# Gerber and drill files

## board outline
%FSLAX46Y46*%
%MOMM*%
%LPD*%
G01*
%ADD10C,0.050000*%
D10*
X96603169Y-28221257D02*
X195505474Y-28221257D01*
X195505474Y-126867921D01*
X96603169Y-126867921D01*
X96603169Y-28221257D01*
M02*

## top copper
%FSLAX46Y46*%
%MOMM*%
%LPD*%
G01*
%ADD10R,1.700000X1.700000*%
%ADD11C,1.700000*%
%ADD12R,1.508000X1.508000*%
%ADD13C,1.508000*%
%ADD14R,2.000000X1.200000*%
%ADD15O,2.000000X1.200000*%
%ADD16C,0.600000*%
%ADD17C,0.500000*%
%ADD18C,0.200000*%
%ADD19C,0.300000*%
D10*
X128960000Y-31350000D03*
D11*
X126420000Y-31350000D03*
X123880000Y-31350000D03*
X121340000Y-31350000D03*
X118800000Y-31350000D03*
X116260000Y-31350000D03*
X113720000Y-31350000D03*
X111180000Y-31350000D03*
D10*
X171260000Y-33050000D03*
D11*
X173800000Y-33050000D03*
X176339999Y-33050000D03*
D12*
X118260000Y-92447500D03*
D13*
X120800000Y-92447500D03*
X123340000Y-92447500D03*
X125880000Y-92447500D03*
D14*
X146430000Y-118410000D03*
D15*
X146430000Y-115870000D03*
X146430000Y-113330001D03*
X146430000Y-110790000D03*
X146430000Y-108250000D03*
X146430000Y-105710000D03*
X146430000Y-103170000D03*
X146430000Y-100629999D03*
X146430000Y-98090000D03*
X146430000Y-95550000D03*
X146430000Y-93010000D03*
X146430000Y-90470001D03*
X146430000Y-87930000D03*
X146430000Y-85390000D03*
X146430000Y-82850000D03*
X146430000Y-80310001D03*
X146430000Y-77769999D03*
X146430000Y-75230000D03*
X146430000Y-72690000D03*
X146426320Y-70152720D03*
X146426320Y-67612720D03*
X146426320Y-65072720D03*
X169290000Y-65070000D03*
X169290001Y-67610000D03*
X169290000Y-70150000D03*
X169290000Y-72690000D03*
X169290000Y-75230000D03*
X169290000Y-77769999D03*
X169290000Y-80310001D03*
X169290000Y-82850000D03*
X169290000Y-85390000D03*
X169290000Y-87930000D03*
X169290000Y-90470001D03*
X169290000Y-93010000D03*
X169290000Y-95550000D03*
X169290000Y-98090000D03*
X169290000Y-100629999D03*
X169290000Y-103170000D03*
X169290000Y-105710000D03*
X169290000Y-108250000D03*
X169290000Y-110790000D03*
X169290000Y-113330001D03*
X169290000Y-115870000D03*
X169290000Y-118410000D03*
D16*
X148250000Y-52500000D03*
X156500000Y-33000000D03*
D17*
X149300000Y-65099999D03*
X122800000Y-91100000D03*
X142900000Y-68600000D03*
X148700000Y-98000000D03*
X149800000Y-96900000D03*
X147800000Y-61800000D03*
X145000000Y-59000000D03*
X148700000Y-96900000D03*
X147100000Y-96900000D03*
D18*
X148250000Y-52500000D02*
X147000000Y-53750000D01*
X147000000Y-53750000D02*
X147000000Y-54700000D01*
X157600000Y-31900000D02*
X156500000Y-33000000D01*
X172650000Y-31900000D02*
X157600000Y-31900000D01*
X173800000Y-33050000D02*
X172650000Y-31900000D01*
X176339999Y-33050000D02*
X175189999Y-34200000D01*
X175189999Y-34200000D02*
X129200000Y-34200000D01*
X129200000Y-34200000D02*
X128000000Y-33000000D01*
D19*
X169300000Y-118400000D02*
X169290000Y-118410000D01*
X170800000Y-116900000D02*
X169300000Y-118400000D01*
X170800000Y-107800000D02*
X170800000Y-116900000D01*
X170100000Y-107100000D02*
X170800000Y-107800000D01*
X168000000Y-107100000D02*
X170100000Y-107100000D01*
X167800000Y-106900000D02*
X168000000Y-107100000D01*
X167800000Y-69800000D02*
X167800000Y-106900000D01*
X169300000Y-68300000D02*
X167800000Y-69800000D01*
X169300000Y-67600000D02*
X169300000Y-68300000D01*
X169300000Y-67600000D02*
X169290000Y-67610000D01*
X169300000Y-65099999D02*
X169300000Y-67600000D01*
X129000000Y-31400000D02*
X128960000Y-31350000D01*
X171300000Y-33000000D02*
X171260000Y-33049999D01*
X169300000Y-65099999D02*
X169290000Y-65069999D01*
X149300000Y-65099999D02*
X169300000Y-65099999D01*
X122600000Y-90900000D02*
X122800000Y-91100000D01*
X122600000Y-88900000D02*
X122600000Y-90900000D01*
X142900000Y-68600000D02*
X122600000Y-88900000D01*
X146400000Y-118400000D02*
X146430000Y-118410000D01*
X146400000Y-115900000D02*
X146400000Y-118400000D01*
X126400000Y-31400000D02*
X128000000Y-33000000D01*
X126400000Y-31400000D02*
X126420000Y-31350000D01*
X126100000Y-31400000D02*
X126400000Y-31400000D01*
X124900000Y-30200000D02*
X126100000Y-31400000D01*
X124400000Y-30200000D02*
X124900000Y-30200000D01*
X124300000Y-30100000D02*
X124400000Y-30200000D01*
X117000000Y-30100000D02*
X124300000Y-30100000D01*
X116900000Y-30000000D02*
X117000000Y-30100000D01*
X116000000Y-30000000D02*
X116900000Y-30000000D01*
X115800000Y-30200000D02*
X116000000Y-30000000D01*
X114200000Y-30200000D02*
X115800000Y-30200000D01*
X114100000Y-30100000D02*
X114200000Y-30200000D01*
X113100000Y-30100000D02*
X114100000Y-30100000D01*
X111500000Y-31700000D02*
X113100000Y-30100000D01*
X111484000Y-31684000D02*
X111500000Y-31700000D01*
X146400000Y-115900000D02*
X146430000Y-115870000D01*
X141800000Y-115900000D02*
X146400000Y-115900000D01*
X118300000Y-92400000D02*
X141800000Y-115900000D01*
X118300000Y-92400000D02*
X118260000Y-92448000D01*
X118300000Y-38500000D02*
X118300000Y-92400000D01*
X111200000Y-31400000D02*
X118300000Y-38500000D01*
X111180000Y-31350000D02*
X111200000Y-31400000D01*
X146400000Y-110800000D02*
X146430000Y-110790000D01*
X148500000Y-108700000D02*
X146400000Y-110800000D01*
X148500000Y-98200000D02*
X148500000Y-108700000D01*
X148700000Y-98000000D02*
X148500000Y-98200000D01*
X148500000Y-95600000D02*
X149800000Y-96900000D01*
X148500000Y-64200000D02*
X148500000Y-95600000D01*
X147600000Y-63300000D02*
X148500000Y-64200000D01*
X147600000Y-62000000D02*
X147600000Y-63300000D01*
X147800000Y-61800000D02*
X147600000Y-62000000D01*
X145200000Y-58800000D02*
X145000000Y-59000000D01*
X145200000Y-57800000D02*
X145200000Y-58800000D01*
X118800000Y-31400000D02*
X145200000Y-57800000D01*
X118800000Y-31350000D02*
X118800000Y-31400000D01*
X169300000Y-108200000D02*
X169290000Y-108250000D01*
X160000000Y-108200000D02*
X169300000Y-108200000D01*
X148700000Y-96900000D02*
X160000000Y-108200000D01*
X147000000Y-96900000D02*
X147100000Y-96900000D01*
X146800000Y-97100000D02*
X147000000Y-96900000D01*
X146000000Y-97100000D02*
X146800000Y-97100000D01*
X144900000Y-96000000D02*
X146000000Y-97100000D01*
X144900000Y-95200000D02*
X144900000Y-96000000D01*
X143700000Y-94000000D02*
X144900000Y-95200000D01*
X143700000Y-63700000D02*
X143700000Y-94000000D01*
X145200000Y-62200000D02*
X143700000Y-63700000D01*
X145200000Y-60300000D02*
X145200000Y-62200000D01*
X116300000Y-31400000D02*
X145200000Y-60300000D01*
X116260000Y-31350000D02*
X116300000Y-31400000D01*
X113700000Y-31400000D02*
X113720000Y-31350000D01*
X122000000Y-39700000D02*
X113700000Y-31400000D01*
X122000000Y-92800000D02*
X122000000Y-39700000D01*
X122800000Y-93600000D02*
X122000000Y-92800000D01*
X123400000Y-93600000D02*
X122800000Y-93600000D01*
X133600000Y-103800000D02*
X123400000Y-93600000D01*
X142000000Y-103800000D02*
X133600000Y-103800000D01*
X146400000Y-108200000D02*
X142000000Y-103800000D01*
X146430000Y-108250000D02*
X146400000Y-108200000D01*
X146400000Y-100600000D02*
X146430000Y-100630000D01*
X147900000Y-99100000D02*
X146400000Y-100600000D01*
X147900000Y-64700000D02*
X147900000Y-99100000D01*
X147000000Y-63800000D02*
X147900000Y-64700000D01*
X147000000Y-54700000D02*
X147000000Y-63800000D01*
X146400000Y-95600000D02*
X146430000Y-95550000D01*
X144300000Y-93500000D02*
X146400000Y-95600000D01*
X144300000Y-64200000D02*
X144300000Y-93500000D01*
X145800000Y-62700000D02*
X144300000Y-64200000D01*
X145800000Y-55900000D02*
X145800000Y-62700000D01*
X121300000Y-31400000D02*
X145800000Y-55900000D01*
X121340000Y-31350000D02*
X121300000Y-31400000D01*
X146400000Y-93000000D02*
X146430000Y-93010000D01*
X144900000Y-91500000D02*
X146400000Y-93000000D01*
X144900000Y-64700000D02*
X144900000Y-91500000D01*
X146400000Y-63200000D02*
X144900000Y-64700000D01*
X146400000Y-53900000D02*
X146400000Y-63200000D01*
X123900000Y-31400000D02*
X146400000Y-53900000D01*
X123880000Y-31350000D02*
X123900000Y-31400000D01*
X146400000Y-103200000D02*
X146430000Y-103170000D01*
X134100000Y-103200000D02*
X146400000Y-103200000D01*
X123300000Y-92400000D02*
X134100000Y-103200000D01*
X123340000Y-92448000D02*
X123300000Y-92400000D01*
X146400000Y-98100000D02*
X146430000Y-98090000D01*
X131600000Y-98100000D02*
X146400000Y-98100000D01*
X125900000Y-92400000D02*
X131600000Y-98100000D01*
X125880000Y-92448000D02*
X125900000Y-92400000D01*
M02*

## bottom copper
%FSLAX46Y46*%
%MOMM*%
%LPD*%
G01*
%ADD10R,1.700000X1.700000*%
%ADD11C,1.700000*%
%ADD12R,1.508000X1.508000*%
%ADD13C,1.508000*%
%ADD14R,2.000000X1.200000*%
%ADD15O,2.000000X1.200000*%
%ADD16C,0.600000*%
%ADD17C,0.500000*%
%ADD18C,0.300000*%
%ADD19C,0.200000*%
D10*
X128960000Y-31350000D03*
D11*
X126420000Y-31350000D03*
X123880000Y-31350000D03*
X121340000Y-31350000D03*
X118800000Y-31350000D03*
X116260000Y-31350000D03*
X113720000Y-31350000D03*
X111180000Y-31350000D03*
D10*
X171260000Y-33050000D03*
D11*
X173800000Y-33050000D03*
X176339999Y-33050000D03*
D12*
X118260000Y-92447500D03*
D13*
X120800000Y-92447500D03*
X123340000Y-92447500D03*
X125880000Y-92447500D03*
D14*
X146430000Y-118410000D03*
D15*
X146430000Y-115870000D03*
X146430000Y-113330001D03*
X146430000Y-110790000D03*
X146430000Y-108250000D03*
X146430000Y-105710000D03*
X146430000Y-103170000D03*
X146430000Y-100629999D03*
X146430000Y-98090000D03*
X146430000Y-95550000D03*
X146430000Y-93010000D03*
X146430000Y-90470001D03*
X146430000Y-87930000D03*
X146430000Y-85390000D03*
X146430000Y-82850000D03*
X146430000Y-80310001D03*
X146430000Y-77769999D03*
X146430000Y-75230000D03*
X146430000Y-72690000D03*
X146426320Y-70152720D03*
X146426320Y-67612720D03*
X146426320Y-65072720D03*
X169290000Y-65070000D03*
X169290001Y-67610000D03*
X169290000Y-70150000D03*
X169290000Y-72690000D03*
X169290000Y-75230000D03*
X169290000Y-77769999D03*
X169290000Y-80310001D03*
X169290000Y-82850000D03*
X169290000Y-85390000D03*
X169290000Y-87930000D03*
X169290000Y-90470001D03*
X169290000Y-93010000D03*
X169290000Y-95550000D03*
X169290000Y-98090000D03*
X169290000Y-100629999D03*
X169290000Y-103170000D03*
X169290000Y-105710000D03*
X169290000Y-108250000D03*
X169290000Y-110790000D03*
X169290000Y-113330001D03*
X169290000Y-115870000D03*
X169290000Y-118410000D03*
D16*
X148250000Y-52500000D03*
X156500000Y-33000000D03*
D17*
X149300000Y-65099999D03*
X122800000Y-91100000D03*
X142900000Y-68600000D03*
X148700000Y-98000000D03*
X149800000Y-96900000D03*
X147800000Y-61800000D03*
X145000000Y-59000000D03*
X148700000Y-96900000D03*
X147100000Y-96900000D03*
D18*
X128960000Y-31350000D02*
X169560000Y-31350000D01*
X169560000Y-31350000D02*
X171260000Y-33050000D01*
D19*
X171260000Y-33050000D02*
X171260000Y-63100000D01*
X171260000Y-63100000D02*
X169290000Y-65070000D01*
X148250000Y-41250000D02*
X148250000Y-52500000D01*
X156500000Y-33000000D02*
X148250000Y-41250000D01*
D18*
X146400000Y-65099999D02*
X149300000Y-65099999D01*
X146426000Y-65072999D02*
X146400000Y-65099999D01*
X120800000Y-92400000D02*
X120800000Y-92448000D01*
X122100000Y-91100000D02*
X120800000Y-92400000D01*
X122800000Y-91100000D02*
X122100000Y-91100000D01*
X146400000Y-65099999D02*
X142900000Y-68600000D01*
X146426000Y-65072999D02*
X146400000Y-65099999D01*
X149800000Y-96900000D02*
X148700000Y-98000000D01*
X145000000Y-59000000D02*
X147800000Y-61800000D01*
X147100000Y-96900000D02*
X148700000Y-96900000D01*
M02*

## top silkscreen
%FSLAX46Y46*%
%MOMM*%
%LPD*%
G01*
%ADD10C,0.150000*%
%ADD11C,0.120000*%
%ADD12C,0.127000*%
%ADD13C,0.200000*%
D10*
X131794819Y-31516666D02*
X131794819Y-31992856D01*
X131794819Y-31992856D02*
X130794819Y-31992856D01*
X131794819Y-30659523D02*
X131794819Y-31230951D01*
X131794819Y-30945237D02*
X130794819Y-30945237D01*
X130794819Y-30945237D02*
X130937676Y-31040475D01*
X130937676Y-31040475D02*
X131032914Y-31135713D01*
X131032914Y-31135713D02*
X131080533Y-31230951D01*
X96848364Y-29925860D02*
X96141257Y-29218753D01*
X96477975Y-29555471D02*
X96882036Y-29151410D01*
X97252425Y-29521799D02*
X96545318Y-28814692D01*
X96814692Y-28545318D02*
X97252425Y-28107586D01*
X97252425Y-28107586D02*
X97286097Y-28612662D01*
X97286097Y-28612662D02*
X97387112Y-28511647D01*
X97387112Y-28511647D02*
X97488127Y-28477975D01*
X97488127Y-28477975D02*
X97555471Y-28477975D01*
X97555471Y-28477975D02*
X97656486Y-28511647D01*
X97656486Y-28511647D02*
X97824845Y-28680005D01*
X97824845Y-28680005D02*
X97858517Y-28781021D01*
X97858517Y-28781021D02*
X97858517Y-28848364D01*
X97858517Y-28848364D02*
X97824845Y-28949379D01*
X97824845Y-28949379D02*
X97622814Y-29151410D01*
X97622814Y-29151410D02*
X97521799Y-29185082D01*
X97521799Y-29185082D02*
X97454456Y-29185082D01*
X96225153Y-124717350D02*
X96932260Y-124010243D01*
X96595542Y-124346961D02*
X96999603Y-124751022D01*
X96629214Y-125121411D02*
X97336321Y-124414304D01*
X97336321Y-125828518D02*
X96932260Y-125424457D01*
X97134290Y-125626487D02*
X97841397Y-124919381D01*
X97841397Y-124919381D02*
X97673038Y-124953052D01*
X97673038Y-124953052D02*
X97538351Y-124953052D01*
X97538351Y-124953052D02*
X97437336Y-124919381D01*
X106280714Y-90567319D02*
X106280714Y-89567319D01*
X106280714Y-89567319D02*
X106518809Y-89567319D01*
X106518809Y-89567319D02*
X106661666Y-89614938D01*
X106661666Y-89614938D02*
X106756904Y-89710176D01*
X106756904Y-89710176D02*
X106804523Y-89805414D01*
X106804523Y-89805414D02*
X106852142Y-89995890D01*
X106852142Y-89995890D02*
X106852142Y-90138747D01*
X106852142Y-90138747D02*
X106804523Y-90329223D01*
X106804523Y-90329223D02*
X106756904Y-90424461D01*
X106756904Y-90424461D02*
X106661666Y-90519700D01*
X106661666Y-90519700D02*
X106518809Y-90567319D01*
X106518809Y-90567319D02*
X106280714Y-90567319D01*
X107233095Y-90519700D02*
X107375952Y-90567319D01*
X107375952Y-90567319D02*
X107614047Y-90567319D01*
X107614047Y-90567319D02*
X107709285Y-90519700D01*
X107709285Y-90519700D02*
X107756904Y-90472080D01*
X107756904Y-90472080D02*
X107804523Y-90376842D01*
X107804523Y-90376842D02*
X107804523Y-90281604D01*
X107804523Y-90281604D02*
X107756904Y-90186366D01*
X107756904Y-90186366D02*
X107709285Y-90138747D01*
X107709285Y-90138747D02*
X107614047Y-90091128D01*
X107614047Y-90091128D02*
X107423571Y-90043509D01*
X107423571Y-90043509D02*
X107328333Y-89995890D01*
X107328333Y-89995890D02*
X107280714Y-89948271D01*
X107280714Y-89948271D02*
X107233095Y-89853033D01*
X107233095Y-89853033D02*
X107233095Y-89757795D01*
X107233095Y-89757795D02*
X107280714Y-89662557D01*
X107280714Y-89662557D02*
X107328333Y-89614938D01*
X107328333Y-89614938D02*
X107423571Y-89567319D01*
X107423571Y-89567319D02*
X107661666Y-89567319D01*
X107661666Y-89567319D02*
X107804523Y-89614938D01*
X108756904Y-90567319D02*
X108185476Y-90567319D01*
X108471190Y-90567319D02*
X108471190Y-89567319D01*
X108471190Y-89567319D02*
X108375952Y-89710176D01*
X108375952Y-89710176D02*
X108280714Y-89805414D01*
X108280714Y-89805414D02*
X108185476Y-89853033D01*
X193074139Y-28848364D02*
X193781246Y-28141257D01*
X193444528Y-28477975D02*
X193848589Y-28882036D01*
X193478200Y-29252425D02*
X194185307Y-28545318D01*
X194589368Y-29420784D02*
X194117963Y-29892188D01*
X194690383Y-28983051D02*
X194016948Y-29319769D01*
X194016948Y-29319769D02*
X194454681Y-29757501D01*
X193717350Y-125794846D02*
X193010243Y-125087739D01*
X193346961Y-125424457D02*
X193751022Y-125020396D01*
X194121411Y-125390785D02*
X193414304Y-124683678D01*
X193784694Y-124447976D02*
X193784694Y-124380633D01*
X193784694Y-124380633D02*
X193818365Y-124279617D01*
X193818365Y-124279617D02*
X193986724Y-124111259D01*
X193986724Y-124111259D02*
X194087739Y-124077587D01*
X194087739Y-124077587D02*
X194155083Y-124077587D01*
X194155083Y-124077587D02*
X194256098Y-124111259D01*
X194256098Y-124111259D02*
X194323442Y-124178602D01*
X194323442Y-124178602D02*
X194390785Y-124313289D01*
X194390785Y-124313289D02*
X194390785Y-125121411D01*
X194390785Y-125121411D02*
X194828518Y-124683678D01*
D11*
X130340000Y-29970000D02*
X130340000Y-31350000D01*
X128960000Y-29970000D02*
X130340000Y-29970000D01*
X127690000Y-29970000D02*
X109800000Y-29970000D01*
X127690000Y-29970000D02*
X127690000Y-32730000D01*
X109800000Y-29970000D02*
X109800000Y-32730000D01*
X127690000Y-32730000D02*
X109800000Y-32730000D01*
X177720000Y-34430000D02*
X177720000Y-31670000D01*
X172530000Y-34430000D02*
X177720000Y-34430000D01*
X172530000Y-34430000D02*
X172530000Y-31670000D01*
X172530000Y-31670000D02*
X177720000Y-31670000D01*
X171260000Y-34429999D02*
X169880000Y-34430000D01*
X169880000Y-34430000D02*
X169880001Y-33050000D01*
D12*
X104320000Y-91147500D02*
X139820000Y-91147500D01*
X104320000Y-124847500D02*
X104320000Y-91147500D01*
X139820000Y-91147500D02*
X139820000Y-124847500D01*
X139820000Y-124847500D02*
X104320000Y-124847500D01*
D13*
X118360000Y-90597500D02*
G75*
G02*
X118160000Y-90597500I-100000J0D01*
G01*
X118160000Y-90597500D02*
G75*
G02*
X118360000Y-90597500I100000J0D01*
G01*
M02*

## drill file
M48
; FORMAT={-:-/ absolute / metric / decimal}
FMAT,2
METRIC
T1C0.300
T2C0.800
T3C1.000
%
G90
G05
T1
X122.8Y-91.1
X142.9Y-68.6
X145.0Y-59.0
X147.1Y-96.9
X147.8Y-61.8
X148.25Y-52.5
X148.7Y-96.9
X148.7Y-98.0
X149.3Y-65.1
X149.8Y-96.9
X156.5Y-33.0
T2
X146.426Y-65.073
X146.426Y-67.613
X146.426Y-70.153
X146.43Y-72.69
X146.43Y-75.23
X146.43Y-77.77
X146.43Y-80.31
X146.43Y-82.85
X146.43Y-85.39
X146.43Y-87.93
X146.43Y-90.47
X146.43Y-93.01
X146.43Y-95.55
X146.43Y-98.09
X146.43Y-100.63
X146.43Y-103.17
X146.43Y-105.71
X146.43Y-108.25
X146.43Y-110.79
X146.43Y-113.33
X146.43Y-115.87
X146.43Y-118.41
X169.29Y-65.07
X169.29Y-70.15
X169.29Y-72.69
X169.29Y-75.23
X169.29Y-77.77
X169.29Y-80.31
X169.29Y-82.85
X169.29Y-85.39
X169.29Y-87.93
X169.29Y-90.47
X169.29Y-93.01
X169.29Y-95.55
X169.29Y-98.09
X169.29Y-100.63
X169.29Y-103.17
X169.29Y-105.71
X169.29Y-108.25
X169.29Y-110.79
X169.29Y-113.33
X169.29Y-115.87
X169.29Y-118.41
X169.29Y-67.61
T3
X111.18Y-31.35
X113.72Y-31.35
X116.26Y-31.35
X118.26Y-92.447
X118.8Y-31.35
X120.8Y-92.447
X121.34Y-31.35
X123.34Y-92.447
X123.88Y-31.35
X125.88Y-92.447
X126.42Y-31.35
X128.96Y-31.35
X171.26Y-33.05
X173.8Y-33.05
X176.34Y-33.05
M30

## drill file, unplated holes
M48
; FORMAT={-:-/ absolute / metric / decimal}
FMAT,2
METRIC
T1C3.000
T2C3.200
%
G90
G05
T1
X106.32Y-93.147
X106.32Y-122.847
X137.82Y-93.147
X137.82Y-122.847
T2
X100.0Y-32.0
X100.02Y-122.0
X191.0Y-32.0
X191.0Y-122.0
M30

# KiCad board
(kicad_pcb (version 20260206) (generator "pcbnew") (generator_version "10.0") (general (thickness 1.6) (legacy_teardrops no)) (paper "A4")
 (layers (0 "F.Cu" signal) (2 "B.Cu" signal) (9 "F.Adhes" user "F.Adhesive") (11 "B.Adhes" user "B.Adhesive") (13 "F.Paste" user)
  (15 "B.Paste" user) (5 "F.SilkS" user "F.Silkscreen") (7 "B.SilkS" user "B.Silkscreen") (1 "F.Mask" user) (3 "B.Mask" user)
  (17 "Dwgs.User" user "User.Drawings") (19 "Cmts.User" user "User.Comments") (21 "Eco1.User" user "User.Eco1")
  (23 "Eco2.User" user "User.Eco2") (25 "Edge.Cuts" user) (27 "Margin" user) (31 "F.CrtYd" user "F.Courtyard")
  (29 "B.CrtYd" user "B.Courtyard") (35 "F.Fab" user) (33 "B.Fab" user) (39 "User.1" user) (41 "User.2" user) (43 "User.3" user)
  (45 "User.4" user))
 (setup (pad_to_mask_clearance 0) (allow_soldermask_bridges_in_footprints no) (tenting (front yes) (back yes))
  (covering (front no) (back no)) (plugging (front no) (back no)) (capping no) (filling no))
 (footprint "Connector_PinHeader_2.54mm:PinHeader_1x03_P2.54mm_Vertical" (layer "F.Cu") (at 171.26 33.05 90)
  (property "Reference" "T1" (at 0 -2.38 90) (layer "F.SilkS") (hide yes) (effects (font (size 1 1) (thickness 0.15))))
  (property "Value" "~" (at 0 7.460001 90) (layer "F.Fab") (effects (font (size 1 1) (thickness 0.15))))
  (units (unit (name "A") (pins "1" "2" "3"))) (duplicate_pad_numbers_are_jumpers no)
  (fp_line (start -1.38 -1.38) (end 0 -1.379999) (stroke (width 0.12) (type solid)) (layer "F.SilkS"))
  (fp_line (start -1.379999 0) (end -1.38 -1.38) (stroke (width 0.12) (type solid)) (layer "F.SilkS"))
  (fp_line (start 1.38 1.27) (end 1.38 6.46) (stroke (width 0.12) (type solid)) (layer "F.SilkS"))
  (fp_line (start -1.38 1.27) (end 1.38 1.27) (stroke (width 0.12) (type solid)) (layer "F.SilkS"))
  (fp_line (start -1.38 1.27) (end -1.38 6.46) (stroke (width 0.12) (type solid)) (layer "F.SilkS"))
  (fp_line (start -1.38 6.46) (end 1.38 6.46) (stroke (width 0.12) (type solid)) (layer "F.SilkS"))
  (pad "1" thru_hole rect (at 0 0 90) (size 1.7 1.7) (drill 1) (layers "*.Cu" "*.Mask") (remove_unused_layers no) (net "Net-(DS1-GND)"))
  (pad "2" thru_hole circle (at 0 2.54 90) (size 1.7 1.7) (drill 1) (layers "*.Cu" "*.Mask") (remove_unused_layers no) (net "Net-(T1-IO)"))
  (pad "3" thru_hole circle (at 0 5.079999 90) (size 1.7 1.7) (drill 1) (layers "*.Cu" "*.Mask") (remove_unused_layers no)
   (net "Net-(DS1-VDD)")))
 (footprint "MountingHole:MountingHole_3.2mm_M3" (layer "F.Cu") (at 100 32 45)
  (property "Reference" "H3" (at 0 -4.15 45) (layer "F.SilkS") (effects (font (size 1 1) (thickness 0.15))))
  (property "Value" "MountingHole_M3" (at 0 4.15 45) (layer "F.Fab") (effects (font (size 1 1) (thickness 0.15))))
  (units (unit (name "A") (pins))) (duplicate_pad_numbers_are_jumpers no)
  (pad "" np_thru_hole circle (at 0 0 45) (size 3.2 3.2) (drill 3.2) (layers "*.Cu" "*.Mask")))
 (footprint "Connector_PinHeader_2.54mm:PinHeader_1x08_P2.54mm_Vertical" (layer "F.Cu") (at 128.96 31.35 -90)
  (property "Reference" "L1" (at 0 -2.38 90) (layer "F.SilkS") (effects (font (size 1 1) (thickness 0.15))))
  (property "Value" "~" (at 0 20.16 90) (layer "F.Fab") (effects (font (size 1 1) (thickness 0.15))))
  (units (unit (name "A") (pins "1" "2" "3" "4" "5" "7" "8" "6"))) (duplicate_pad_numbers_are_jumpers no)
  (fp_line (start -1.38 19.16) (end 1.38 19.16) (stroke (width 0.12) (type solid)) (layer "F.SilkS"))
  (fp_line (start -1.38 1.27) (end -1.38 19.16) (stroke (width 0.12) (type solid)) (layer "F.SilkS"))
  (fp_line (start -1.38 1.27) (end 1.38 1.27) (stroke (width 0.12) (type solid)) (layer "F.SilkS"))
  (fp_line (start 1.38 1.27) (end 1.38 19.16) (stroke (width 0.12) (type solid)) (layer "F.SilkS"))
  (fp_line (start -1.38 0) (end -1.38 -1.38) (stroke (width 0.12) (type solid)) (layer "F.SilkS"))
  (fp_line (start -1.38 -1.38) (end 0 -1.38) (stroke (width 0.12) (type solid)) (layer "F.SilkS"))
  (pad "1" thru_hole rect (at 0 0 270) (size 1.7 1.7) (drill 1) (layers "*.Cu" "*.Mask") (remove_unused_layers no) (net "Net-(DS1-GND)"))
  (pad "2" thru_hole circle (at 0 2.54 270) (size 1.7 1.7) (drill 1) (layers "*.Cu" "*.Mask") (remove_unused_layers no)
   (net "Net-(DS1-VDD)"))
  (pad "3" thru_hole circle (at 0 5.08 270) (size 1.7 1.7) (drill 1) (layers "*.Cu" "*.Mask") (remove_unused_layers no) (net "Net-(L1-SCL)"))
  (pad "4" thru_hole circle (at 0 7.62 270) (size 1.7 1.7) (drill 1) (layers "*.Cu" "*.Mask") (remove_unused_layers no) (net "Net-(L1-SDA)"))
  (pad "5" thru_hole circle (at 0 10.16 270) (size 1.7 1.7) (drill 1) (layers "*.Cu" "*.Mask") (remove_unused_layers no)
   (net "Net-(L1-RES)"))
  (pad "6" thru_hole circle (at 0 12.7 270) (size 1.7 1.7) (drill 1) (layers "*.Cu" "*.Mask") (remove_unused_layers no) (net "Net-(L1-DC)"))
  (pad "7" thru_hole circle (at 0 15.24 270) (size 1.7 1.7) (drill 1) (layers "*.Cu" "*.Mask") (remove_unused_layers no) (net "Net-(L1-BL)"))
  (pad "8" thru_hole circle (at 0 17.78 270) (size 1.7 1.7) (drill 1) (layers "*.Cu" "*.Mask") (remove_unused_layers no)
   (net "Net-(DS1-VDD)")))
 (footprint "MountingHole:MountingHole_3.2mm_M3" (layer "F.Cu") (at 100.02 122 135)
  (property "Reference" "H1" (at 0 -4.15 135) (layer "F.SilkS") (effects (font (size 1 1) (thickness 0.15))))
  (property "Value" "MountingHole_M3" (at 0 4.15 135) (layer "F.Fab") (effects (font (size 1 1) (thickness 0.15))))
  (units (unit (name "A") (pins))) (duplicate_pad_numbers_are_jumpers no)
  (pad "" np_thru_hole circle (at 0 0 135) (size 3.2 3.2) (drill 3.2) (layers "*.Cu" "*.Mask")))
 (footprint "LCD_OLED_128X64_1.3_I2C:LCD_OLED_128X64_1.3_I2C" (layer "F.Cu") (at 122.07 107.9975)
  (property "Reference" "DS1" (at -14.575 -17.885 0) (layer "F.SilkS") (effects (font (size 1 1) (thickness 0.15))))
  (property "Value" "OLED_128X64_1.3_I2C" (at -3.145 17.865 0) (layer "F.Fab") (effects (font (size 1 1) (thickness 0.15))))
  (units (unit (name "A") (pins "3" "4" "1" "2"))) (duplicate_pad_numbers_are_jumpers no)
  (fp_line (start -17.75 -16.85) (end 17.75 -16.85) (stroke (width 0.127) (type solid)) (layer "F.SilkS"))
  (fp_line (start -17.75 16.85) (end -17.75 -16.85) (stroke (width 0.127) (type solid)) (layer "F.SilkS"))
  (fp_line (start 17.75 -16.85) (end 17.75 16.85) (stroke (width 0.127) (type solid)) (layer "F.SilkS"))
  (fp_line (start 17.75 16.85) (end -17.75 16.85) (stroke (width 0.127) (type solid)) (layer "F.SilkS"))
  (fp_circle (center -3.81 -17.4) (end -3.71 -17.4) (stroke (width 0.2) (type solid)) (fill no) (layer "F.SilkS"))
  (pad "" np_thru_hole circle (at -15.75 -14.85) (size 3 3) (drill 3) (layers "*.Cu" "*.Mask"))
  (pad "" np_thru_hole circle (at -15.75 14.85) (size 3 3) (drill 3) (layers "*.Cu" "*.Mask"))
  (pad "" np_thru_hole circle (at 15.75 -14.85) (size 3 3) (drill 3) (layers "*.Cu" "*.Mask"))
  (pad "" np_thru_hole circle (at 15.75 14.85) (size 3 3) (drill 3) (layers "*.Cu" "*.Mask"))
  (pad "1" thru_hole rect (at -3.81 -15.55) (size 1.508 1.508) (drill 1) (layers "*.Cu" "*.Mask") (remove_unused_layers no)
   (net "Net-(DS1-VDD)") (solder_mask_margin 0.102))
  (pad "2" thru_hole circle (at -1.27 -15.55) (size 1.508 1.508) (drill 1) (layers "*.Cu" "*.Mask") (remove_unused_layers no)
   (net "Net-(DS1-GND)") (solder_mask_margin 0.102))
  (pad "3" thru_hole circle (at 1.27 -15.55) (size 1.508 1.508) (drill 1) (layers "*.Cu" "*.Mask") (remove_unused_layers no)
   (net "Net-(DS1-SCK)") (solder_mask_margin 0.102))
  (pad "4" thru_hole circle (at 3.81 -15.55) (size 1.508 1.508) (drill 1) (layers "*.Cu" "*.Mask") (remove_unused_layers no)
   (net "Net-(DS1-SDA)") (solder_mask_margin 0.102)))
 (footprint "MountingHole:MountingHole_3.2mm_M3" (layer "F.Cu") (at 191 32 -45)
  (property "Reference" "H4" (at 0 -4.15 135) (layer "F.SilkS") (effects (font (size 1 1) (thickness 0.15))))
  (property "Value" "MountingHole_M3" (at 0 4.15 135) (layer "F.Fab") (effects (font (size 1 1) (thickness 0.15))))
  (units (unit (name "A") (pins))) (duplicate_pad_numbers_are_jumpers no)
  (pad "" np_thru_hole circle (at 0 0 315) (size 3.2 3.2) (drill 3.2) (layers "*.Cu" "*.Mask")))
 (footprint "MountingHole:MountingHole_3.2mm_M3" (layer "F.Cu") (at 191 122 -135)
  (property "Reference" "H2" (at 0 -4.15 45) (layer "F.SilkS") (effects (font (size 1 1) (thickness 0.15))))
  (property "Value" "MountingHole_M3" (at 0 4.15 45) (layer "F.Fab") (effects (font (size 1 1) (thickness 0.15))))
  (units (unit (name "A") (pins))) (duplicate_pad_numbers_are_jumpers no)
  (pad "" np_thru_hole circle (at 0 0 225) (size 3.2 3.2) (drill 3.2) (layers "*.Cu" "*.Mask")))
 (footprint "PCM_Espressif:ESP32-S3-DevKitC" (layer "B.Cu") (at 146.43 118.41)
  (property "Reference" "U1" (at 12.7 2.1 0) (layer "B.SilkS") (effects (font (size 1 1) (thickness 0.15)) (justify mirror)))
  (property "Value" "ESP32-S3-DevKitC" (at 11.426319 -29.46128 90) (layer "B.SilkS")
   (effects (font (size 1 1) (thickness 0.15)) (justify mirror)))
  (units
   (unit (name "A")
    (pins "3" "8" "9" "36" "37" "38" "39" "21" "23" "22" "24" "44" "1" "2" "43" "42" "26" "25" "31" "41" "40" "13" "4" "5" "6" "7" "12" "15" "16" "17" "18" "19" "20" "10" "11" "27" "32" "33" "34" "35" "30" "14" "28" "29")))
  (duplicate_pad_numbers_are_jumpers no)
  (pad "1" thru_hole rect (at 0 0 90) (size 1.2 2) (drill 0.8) (layers "*.Cu" "*.Mask") (remove_unused_layers no) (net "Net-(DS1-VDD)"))
  (pad "2" thru_hole oval (at 0 -2.54 90) (size 1.2 2) (drill 0.8) (layers "*.Cu" "*.Mask") (remove_unused_layers no) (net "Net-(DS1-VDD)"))
  (pad "3" thru_hole oval (at 0 -5.079999 90) (size 1.2 2) (drill 0.8) (layers "*.Cu" "*.Mask") (remove_unused_layers no)
   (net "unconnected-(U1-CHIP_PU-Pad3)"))
  (pad "4" thru_hole oval (at 0 -7.62 90) (size 1.2 2) (drill 0.8) (layers "*.Cu" "*.Mask") (remove_unused_layers no) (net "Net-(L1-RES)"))
  (pad "5" thru_hole oval (at 0 -10.16 90) (size 1.2 2) (drill 0.8) (layers "*.Cu" "*.Mask") (remove_unused_layers no) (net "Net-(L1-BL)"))
  (pad "6" thru_hole oval (at 0 -12.7 90) (size 1.2 2) (drill 0.8) (layers "*.Cu" "*.Mask") (remove_unused_layers no)
   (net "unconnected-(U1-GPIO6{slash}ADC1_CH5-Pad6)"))
  (pad "7" thru_hole oval (at 0 -15.24 90) (size 1.2 2) (drill 0.8) (layers "*.Cu" "*.Mask") (remove_unused_layers no) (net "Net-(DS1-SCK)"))
  (pad "8" thru_hole oval (at 0 -17.780001 90) (size 1.2 2) (drill 0.8) (layers "*.Cu" "*.Mask") (remove_unused_layers no)
   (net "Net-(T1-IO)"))
  (pad "9" thru_hole oval (at 0 -20.32 90) (size 1.2 2) (drill 0.8) (layers "*.Cu" "*.Mask") (remove_unused_layers no) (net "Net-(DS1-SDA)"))
  (pad "10" thru_hole oval (at 0 -22.86 90) (size 1.2 2) (drill 0.8) (layers "*.Cu" "*.Mask") (remove_unused_layers no) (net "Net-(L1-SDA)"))
  (pad "11" thru_hole oval (at 0 -25.4 90) (size 1.2 2) (drill 0.8) (layers "*.Cu" "*.Mask") (remove_unused_layers no) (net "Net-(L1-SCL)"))
  (pad "12" thru_hole oval (at 0 -27.939999 90) (size 1.2 2) (drill 0.8) (layers "*.Cu" "*.Mask") (remove_unused_layers no)
   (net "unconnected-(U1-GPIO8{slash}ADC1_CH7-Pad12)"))
  (pad "13" thru_hole oval (at 0 -30.48 90) (size 1.2 2) (drill 0.8) (layers "*.Cu" "*.Mask") (remove_unused_layers no)
   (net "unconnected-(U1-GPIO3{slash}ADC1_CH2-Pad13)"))
  (pad "14" thru_hole oval (at 0 -33.02 90) (size 1.2 2) (drill 0.8) (layers "*.Cu" "*.Mask") (remove_unused_layers no)
   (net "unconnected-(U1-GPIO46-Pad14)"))
  (pad "15" thru_hole oval (at 0 -35.56 90) (size 1.2 2) (drill 0.8) (layers "*.Cu" "*.Mask") (remove_unused_layers no)
   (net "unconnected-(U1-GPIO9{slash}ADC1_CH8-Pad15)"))
  (pad "16" thru_hole oval (at 0 -38.099999 90) (size 1.2 2) (drill 0.8) (layers "*.Cu" "*.Mask") (remove_unused_layers no)
   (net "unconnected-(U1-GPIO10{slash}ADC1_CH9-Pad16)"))
  (pad "17" thru_hole oval (at 0 -40.640001 90) (size 1.2 2) (drill 0.8) (layers "*.Cu" "*.Mask") (remove_unused_layers no)
   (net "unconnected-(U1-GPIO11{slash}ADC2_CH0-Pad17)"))
  (pad "18" thru_hole oval (at 0 -43.18 90) (size 1.2 2) (drill 0.8) (layers "*.Cu" "*.Mask") (remove_unused_layers no)
   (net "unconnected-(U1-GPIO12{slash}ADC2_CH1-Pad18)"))
  (pad "19" thru_hole oval (at 0 -45.72 90) (size 1.2 2) (drill 0.8) (layers "*.Cu" "*.Mask") (remove_unused_layers no)
   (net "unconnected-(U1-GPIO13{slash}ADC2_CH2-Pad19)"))
  (pad "20" thru_hole oval (at -0.00368 -48.25728 90) (size 1.2 2) (drill 0.8) (layers "*.Cu" "*.Mask") (remove_unused_layers no)
   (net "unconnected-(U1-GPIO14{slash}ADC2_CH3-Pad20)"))
  (pad "21" thru_hole oval (at -0.00368 -50.79728 90) (size 1.2 2) (drill 0.8) (layers "*.Cu" "*.Mask") (remove_unused_layers no)
   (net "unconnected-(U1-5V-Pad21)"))
  (pad "22" thru_hole oval (at -0.00368 -53.33728 90) (size 1.2 2) (drill 0.8) (layers "*.Cu" "*.Mask") (remove_unused_layers no)
   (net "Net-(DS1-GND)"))
  (pad "23" thru_hole oval (at 22.86 -53.34 90) (size 1.2 2) (drill 0.8) (layers "*.Cu" "*.Mask") (remove_unused_layers no)
   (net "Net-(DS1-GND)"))
  (pad "24" thru_hole oval (at 22.860001 -50.8 90) (size 1.2 2) (drill 0.8) (layers "*.Cu" "*.Mask") (remove_unused_layers no)
   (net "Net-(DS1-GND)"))
  (pad "25" thru_hole oval (at 22.86 -48.26 90) (size 1.2 2) (drill 0.8) (layers "*.Cu" "*.Mask") (remove_unused_layers no)
   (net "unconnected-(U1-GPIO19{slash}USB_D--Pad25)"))
  (pad "26" thru_hole oval (at 22.86 -45.72 90) (size 1.2 2) (drill 0.8) (layers "*.Cu" "*.Mask") (remove_unused_layers no)
   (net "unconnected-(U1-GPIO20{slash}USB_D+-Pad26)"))
  (pad "27" thru_hole oval (at 22.86 -43.18 90) (size 1.2 2) (drill 0.8) (layers "*.Cu" "*.Mask") (remove_unused_layers no)
   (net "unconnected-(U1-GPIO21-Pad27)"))
  (pad "28" thru_hole oval (at 22.86 -40.640001 90) (size 1.2 2) (drill 0.8) (layers "*.Cu" "*.Mask") (remove_unused_layers no)
   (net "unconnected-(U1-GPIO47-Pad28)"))
  (pad "29" thru_hole oval (at 22.86 -38.099999 90) (size 1.2 2) (drill 0.8) (layers "*.Cu" "*.Mask") (remove_unused_layers no)
   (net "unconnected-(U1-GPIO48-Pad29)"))
  (pad "30" thru_hole oval (at 22.86 -35.56 90) (size 1.2 2) (drill 0.8) (layers "*.Cu" "*.Mask") (remove_unused_layers no)
   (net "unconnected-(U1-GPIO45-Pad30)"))
  (pad "31" thru_hole oval (at 22.86 -33.02 90) (size 1.2 2) (drill 0.8) (layers "*.Cu" "*.Mask") (remove_unused_layers no)
   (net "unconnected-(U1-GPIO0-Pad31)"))
  (pad "32" thru_hole oval (at 22.86 -30.48 90) (size 1.2 2) (drill 0.8) (layers "*.Cu" "*.Mask") (remove_unused_layers no)
   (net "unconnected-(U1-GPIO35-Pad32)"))
  (pad "33" thru_hole oval (at 22.86 -27.939999 90) (size 1.2 2) (drill 0.8) (layers "*.Cu" "*.Mask") (remove_unused_layers no)
   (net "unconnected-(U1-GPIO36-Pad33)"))
  (pad "34" thru_hole oval (at 22.86 -25.4 90) (size 1.2 2) (drill 0.8) (layers "*.Cu" "*.Mask") (remove_unused_layers no)
   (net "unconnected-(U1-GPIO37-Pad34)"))
  (pad "35" thru_hole oval (at 22.86 -22.86 90) (size 1.2 2) (drill 0.8) (layers "*.Cu" "*.Mask") (remove_unused_layers no)
   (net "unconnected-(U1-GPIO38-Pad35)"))
  (pad "36" thru_hole oval (at 22.86 -20.32 90) (size 1.2 2) (drill 0.8) (layers "*.Cu" "*.Mask") (remove_unused_layers no)
   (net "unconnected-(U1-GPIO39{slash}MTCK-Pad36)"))
  (pad "37" thru_hole oval (at 22.86 -17.780001 90) (size 1.2 2) (drill 0.8) (layers "*.Cu" "*.Mask") (remove_unused_layers no)
   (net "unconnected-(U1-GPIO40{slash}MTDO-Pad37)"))
  (pad "38" thru_hole oval (at 22.86 -15.24 90) (size 1.2 2) (drill 0.8) (layers "*.Cu" "*.Mask") (remove_unused_layers no)
   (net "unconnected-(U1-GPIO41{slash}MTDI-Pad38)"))
  (pad "39" thru_hole oval (at 22.86 -12.7 90) (size 1.2 2) (drill 0.8) (layers "*.Cu" "*.Mask") (remove_unused_layers no)
   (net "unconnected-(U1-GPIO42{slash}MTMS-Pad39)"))
  (pad "40" thru_hole oval (at 22.86 -10.16 90) (size 1.2 2) (drill 0.8) (layers "*.Cu" "*.Mask") (remove_unused_layers no)
   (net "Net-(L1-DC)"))
  (pad "41" thru_hole oval (at 22.86 -7.62 90) (size 1.2 2) (drill 0.8) (layers "*.Cu" "*.Mask") (remove_unused_layers no)
   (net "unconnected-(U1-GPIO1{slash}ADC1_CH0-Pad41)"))
  (pad "42" thru_hole oval (at 22.86 -5.079999 90) (size 1.2 2) (drill 0.8) (layers "*.Cu" "*.Mask") (remove_unused_layers no)
   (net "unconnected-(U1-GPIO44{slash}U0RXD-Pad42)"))
  (pad "43" thru_hole oval (at 22.86 -2.54 90) (size 1.2 2) (drill 0.8) (layers "*.Cu" "*.Mask") (remove_unused_layers no)
   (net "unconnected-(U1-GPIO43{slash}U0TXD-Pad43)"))
  (pad "44" thru_hole oval (at 22.86 0 90) (size 1.2 2) (drill 0.8) (layers "*.Cu" "*.Mask") (remove_unused_layers no) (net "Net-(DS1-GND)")))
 (gr_rect (start 96.603169 28.221257) (end 195.505474 126.867921) (stroke (width 0.05) (type default)) (fill no) (layer "Edge.Cuts"))
 (segment (start 122.6 88.9) (end 122.6 90.9) (width 0.3) (layer "F.Cu") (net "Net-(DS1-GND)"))
 (segment (start 129 31.4) (end 128.96 31.35) (width 0.3) (layer "F.Cu") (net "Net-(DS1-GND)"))
 (segment (start 167.8 106.9) (end 168 107.1) (width 0.3) (layer "F.Cu") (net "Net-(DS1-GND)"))
 (segment (start 169.3 118.4) (end 169.29 118.41) (width 0.3) (layer "F.Cu") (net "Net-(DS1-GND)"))
 (segment (start 142.9 68.6) (end 122.6 88.9) (width 0.3) (layer "F.Cu") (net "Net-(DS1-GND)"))
 (segment (start 170.8 107.8) (end 170.8 116.9) (width 0.3) (layer "F.Cu") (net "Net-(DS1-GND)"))
 (segment (start 171.3 33) (end 171.26 33.049999) (width 0.3) (layer "F.Cu") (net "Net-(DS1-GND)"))
 (segment (start 167.8 69.8) (end 167.8 106.9) (width 0.3) (layer "F.Cu") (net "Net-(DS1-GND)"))
 (segment (start 169.3 67.6) (end 169.3 68.3) (width 0.3) (layer "F.Cu") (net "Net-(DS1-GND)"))
 (segment (start 170.8 116.9) (end 169.3 118.4) (width 0.3) (layer "F.Cu") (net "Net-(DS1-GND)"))
 (segment (start 170.1 107.1) (end 170.8 107.8) (width 0.3) (layer "F.Cu") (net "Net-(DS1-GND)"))
 (segment (start 169.3 65.099999) (end 169.29 65.069999) (width 0.3) (layer "F.Cu") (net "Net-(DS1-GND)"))
 (segment (start 168 107.1) (end 170.1 107.1) (width 0.3) (layer "F.Cu") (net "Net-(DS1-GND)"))
 (segment (start 169.3 65.099999) (end 169.3 67.6) (width 0.3) (layer "F.Cu") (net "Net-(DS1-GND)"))
 (segment (start 169.3 68.3) (end 167.8 69.8) (width 0.3) (layer "F.Cu") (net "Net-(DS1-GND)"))
 (segment (start 169.3 67.6) (end 169.29 67.61) (width 0.3) (layer "F.Cu") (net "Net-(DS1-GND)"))
 (segment (start 122.6 90.9) (end 122.8 91.1) (width 0.3) (layer "F.Cu") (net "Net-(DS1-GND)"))
 (segment (start 149.3 65.099999) (end 169.3 65.099999) (width 0.3) (layer "F.Cu") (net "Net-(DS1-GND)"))
 (via (at 142.9 68.6) (size 0.5) (drill 0.3) (layers "F.Cu" "B.Cu") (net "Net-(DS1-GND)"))
 (via (at 122.8 91.1) (size 0.5) (drill 0.3) (layers "F.Cu" "B.Cu") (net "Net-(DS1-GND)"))
 (via (at 149.3 65.099999) (size 0.5) (drill 0.3) (layers "F.Cu" "B.Cu") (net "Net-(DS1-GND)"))
 (segment (start 171.26 33.05) (end 171.26 63.1) (width 0.2) (layer "B.Cu") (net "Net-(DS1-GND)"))
 (segment (start 146.4 65.099999) (end 149.3 65.099999) (width 0.3) (layer "B.Cu") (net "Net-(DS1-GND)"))
 (segment (start 169.56 31.35) (end 171.26 33.05) (width 0.3) (layer "B.Cu") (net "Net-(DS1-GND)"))
 (segment (start 128.96 31.35) (end 169.56 31.35) (width 0.3) (layer "B.Cu") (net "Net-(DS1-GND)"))
 (segment (start 120.8 92.4) (end 120.8 92.448) (width 0.3) (layer "B.Cu") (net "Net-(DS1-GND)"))
 (segment (start 122.1 91.1) (end 120.8 92.4) (width 0.3) (layer "B.Cu") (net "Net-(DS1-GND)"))
 (segment (start 146.426 65.072999) (end 146.4 65.099999) (width 0.3) (layer "B.Cu") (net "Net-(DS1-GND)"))
 (segment (start 171.26 63.1) (end 169.29 65.07) (width 0.2) (layer "B.Cu") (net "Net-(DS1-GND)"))
 (segment (start 146.426 65.072999) (end 146.4 65.099999) (width 0.3) (layer "B.Cu") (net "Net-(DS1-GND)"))
 (segment (start 146.4 65.099999) (end 142.9 68.6) (width 0.3) (layer "B.Cu") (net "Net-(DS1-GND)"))
 (segment (start 122.8 91.1) (end 122.1 91.1) (width 0.3) (layer "B.Cu") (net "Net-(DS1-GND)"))
 (segment (start 148.25 52.5) (end 147 53.75) (width 0.2) (layer "F.Cu") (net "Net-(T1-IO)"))
 (segment (start 147 53.75) (end 147 54.7) (width 0.2) (layer "F.Cu") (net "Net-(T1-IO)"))
 (segment (start 146.4 100.6) (end 146.43 100.63) (width 0.3) (layer "F.Cu") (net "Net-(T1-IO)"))
 (segment (start 157.6 31.9) (end 156.5 33) (width 0.2) (layer "F.Cu") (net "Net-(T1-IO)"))
 (segment (start 147.9 64.7) (end 147.9 99.1) (width 0.3) (layer "F.Cu") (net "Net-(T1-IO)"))
 (segment (start 147 54.7) (end 147 63.8) (width 0.3) (layer "F.Cu") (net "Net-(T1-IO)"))
 (segment (start 172.65 31.9) (end 157.6 31.9) (width 0.2) (layer "F.Cu") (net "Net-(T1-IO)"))
 (segment (start 173.8 33.05) (end 172.65 31.9) (width 0.2) (layer "F.Cu") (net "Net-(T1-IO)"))
 (segment (start 147.9 99.1) (end 146.4 100.6) (width 0.3) (layer "F.Cu") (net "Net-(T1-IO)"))
 (segment (start 147 63.8) (end 147.9 64.7) (width 0.3) (layer "F.Cu") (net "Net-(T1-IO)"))
 (via (at 156.5 33) (size 0.6) (drill 0.3) (layers "F.Cu" "B.Cu") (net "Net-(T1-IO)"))
 (via (at 148.25 52.5) (size 0.6) (drill 0.3) (layers "F.Cu" "B.Cu") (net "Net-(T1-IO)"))
 (segment (start 148.25 41.25) (end 148.25 52.5) (width 0.2) (layer "B.Cu") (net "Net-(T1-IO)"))
 (segment (start 156.5 33) (end 148.25 41.25) (width 0.2) (layer "B.Cu") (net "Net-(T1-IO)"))
 (segment (start 111.2 31.4) (end 118.3 38.5) (width 0.3) (layer "F.Cu") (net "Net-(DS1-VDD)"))
 (segment (start 114.2 30.2) (end 115.8 30.2) (width 0.3) (layer "F.Cu") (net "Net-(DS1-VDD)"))
 (segment (start 116.9 30) (end 117 30.1) (width 0.3) (layer "F.Cu") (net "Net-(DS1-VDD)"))
 (segment (start 116 30) (end 116.9 30) (width 0.3) (layer "F.Cu") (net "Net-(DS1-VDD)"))
 (segment (start 146.4 115.9) (end 146.43 115.87) (width 0.3) (layer "F.Cu") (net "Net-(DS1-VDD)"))
 (segment (start 126.1 31.4) (end 126.4 31.4) (width 0.3) (layer "F.Cu") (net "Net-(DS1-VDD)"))
 (segment (start 146.4 115.9) (end 146.4 118.4) (width 0.3) (layer "F.Cu") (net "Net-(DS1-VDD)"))
 (segment (start 175.189999 34.2) (end 129.2 34.2) (width 0.2) (layer "F.Cu") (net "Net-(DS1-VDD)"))
 (segment (start 114.1 30.1) (end 114.2 30.2) (width 0.3) (layer "F.Cu") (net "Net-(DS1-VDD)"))
 (segment (start 118.3 92.4) (end 141.8 115.9) (width 0.3) (layer "F.Cu") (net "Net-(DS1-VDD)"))
 (segment (start 129.2 34.2) (end 128 33) (width 0.2) (layer "F.Cu") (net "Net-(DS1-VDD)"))
 (segment (start 124.4 30.2) (end 124.9 30.2) (width 0.3) (layer "F.Cu") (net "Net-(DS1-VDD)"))
 (segment (start 124.9 30.2) (end 126.1 31.4) (width 0.3) (layer "F.Cu") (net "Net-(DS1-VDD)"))
 (segment (start 176.339999 33.05) (end 175.189999 34.2) (width 0.2) (layer "F.Cu") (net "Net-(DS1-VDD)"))
 (segment (start 113.1 30.1) (end 114.1 30.1) (width 0.3) (layer "F.Cu") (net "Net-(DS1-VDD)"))
 (segment (start 146.4 118.4) (end 146.43 118.41) (width 0.3) (layer "F.Cu") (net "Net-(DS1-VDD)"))
 (segment (start 126.4 31.4) (end 126.42 31.35) (width 0.3) (layer "F.Cu") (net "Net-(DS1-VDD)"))
 (segment (start 118.3 38.5) (end 118.3 92.4) (width 0.3) (layer "F.Cu") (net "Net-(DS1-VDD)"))
 (segment (start 141.8 115.9) (end 146.4 115.9) (width 0.3) (layer "F.Cu") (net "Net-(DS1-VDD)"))
 (segment (start 117 30.1) (end 124.3 30.1) (width 0.3) (layer "F.Cu") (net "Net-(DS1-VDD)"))
 (segment (start 118.3 92.4) (end 118.26 92.448) (width 0.3) (layer "F.Cu") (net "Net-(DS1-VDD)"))
 (segment (start 124.3 30.1) (end 124.4 30.2) (width 0.3) (layer "F.Cu") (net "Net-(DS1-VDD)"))
 (segment (start 111.5 31.7) (end 113.1 30.1) (width 0.3) (layer "F.Cu") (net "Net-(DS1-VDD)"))
 (segment (start 111.18 31.35) (end 111.2 31.4) (width 0.3) (layer "F.Cu") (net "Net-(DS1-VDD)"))
 (segment (start 111.484 31.684) (end 111.5 31.7) (width 0.3) (layer "F.Cu") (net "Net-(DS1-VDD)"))
 (segment (start 115.8 30.2) (end 116 30) (width 0.3) (layer "F.Cu") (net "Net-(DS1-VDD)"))
 (segment (start 126.4 31.4) (end 128 33) (width 0.3) (layer "F.Cu") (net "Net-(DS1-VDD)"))
 (segment (start 123.9 31.4) (end 146.4 53.9) (width 0.3) (layer "F.Cu") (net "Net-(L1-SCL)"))
 (segment (start 144.9 64.7) (end 144.9 91.5) (width 0.3) (layer "F.Cu") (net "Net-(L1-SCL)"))
 (segment (start 123.88 31.35) (end 123.9 31.4) (width 0.3) (layer "F.Cu") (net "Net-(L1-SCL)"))
 (segment (start 146.4 63.2) (end 144.9 64.7) (width 0.3) (layer "F.Cu") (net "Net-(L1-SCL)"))
 (segment (start 146.4 53.9) (end 146.4 63.2) (width 0.3) (layer "F.Cu") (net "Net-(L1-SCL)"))
 (segment (start 144.9 91.5) (end 146.4 93) (width 0.3) (layer "F.Cu") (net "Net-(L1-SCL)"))
 (segment (start 146.4 93) (end 146.43 93.01) (width 0.3) (layer "F.Cu") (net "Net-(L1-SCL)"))
 (segment (start 121.34 31.35) (end 121.3 31.4) (width 0.3) (layer "F.Cu") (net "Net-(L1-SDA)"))
 (segment (start 144.3 93.5) (end 146.4 95.6) (width 0.3) (layer "F.Cu") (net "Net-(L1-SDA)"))
 (segment (start 146.4 95.6) (end 146.43 95.55) (width 0.3) (layer "F.Cu") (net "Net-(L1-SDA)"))
 (segment (start 121.3 31.4) (end 145.8 55.9) (width 0.3) (layer "F.Cu") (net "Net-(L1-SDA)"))
 (segment (start 144.3 64.2) (end 144.3 93.5) (width 0.3) (layer "F.Cu") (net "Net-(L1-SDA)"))
 (segment (start 145.8 62.7) (end 144.3 64.2) (width 0.3) (layer "F.Cu") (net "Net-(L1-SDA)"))
 (segment (start 145.8 55.9) (end 145.8 62.7) (width 0.3) (layer "F.Cu") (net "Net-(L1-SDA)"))
 (segment (start 145.2 58.8) (end 145 59) (width 0.3) (layer "F.Cu") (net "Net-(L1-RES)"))
 (segment (start 118.8 31.35) (end 118.8 31.4) (width 0.3) (layer "F.Cu") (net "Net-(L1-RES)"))
 (segment (start 148.5 98.2) (end 148.5 108.7) (width 0.3) (layer "F.Cu") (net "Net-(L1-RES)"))
 (segment (start 118.8 31.4) (end 145.2 57.8) (width 0.3) (layer "F.Cu") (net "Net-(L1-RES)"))
 (segment (start 147.8 61.8) (end 147.6 62) (width 0.3) (layer "F.Cu") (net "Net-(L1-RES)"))
 (segment (start 147.6 62) (end 147.6 63.3) (width 0.3) (layer "F.Cu") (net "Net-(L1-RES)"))
 (segment (start 148.7 98) (end 148.5 98.2) (width 0.3) (layer "F.Cu") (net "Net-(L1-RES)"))
 (segment (start 148.5 108.7) (end 146.4 110.8) (width 0.3) (layer "F.Cu") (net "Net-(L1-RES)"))
 (segment (start 147.6 63.3) (end 148.5 64.2) (width 0.3) (layer "F.Cu") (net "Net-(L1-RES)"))
 (segment (start 148.5 64.2) (end 148.5 95.6) (width 0.3) (layer "F.Cu") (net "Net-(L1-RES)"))
 (segment (start 145.2 57.8) (end 145.2 58.8) (width 0.3) (layer "F.Cu") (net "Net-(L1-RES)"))
 (segment (start 148.5 95.6) (end 149.8 96.9) (width 0.3) (layer "F.Cu") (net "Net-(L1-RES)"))
 (segment (start 146.4 110.8) (end 146.43 110.79) (width 0.3) (layer "F.Cu") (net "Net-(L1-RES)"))
 (via (at 148.7 98) (size 0.5) (drill 0.3) (layers "F.Cu" "B.Cu") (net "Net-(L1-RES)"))
 (via (at 149.8 96.9) (size 0.5) (drill 0.3) (layers "F.Cu" "B.Cu") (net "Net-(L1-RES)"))
 (via (at 145 59) (size 0.5) (drill 0.3) (layers "F.Cu" "B.Cu") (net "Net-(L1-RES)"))
 (via (at 147.8 61.8) (size 0.5) (drill 0.3) (layers "F.Cu" "B.Cu") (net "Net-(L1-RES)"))
 (segment (start 149.8 96.9) (end 148.7 98) (width 0.3) (layer "B.Cu") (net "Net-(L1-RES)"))
 (segment (start 145 59) (end 147.8 61.8) (width 0.3) (layer "B.Cu") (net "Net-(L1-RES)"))
 (segment (start 146.4 103.2) (end 146.43 103.17) (width 0.3) (layer "F.Cu") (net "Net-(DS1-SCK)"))
 (segment (start 134.1 103.2) (end 146.4 103.2) (width 0.3) (layer "F.Cu") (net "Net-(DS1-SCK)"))
 (segment (start 123.3 92.4) (end 134.1 103.2) (width 0.3) (layer "F.Cu") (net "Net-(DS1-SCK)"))
 (segment (start 123.34 92.448) (end 123.3 92.4) (width 0.3) (layer "F.Cu") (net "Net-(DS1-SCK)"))
 (segment (start 131.6 98.1) (end 146.4 98.1) (width 0.3) (layer "F.Cu") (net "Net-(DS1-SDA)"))
 (segment (start 125.88 92.448) (end 125.9 92.4) (width 0.3) (layer "F.Cu") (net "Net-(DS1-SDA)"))
 (segment (start 125.9 92.4) (end 131.6 98.1) (width 0.3) (layer "F.Cu") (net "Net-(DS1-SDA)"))
 (segment (start 146.4 98.1) (end 146.43 98.09) (width 0.3) (layer "F.Cu") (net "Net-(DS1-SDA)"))
 (segment (start 133.6 103.8) (end 123.4 93.6) (width 0.3) (layer "F.Cu") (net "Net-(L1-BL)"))
 (segment (start 123.4 93.6) (end 122.8 93.6) (width 0.3) (layer "F.Cu") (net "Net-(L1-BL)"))
 (segment (start 113.7 31.4) (end 113.72 31.35) (width 0.3) (layer "F.Cu") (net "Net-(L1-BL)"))
 (segment (start 122.8 93.6) (end 122 92.8) (width 0.3) (layer "F.Cu") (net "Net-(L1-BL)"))
 (segment (start 146.43 108.25) (end 146.4 108.2) (width 0.3) (layer "F.Cu") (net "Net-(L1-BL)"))
 (segment (start 122 39.7) (end 113.7 31.4) (width 0.3) (layer "F.Cu") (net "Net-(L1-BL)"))
 (segment (start 142 103.8) (end 133.6 103.8) (width 0.3) (layer "F.Cu") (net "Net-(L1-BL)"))
 (segment (start 146.4 108.2) (end 142 103.8) (width 0.3) (layer "F.Cu") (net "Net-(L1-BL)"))
 (segment (start 122 92.8) (end 122 39.7) (width 0.3) (layer "F.Cu") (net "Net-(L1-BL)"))
 (segment (start 144.9 96) (end 146 97.1) (width 0.3) (layer "F.Cu") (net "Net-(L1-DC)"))
 (segment (start 144.9 95.2) (end 144.9 96) (width 0.3) (layer "F.Cu") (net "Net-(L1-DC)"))
 (segment (start 145.2 62.2) (end 143.7 63.7) (width 0.3) (layer "F.Cu") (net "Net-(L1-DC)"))
 (segment (start 143.7 94) (end 144.9 95.2) (width 0.3) (layer "F.Cu") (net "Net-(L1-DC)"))
 (segment (start 146 97.1) (end 146.8 97.1) (width 0.3) (layer "F.Cu") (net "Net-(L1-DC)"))
 (segment (start 148.7 96.9) (end 160 108.2) (width 0.3) (layer "F.Cu") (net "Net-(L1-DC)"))
 (segment (start 147 96.9) (end 147.1 96.9) (width 0.3) (layer "F.Cu") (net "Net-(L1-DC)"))
 (segment (start 116.3 31.4) (end 145.2 60.3) (width 0.3) (layer "F.Cu") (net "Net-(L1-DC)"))
 (segment (start 143.7 63.7) (end 143.7 94) (width 0.3) (layer "F.Cu") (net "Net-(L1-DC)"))
 (segment (start 145.2 60.3) (end 145.2 62.2) (width 0.3) (layer "F.Cu") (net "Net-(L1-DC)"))
 (segment (start 116.26 31.35) (end 116.3 31.4) (width 0.3) (layer "F.Cu") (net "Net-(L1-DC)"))
 (segment (start 169.3 108.2) (end 169.29 108.25) (width 0.3) (layer "F.Cu") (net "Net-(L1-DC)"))
 (segment (start 160 108.2) (end 169.3 108.2) (width 0.3) (layer "F.Cu") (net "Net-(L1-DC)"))
 (segment (start 146.8 97.1) (end 147 96.9) (width 0.3) (layer "F.Cu") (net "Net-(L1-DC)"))
 (via (at 148.7 96.9) (size 0.5) (drill 0.3) (layers "F.Cu" "B.Cu") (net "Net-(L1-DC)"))
 (via (at 147.1 96.9) (size 0.5) (drill 0.3) (layers "F.Cu" "B.Cu") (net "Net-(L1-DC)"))
 (segment (start 147.1 96.9) (end 148.7 96.9) (width 0.3) (layer "B.Cu") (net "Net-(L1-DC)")))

